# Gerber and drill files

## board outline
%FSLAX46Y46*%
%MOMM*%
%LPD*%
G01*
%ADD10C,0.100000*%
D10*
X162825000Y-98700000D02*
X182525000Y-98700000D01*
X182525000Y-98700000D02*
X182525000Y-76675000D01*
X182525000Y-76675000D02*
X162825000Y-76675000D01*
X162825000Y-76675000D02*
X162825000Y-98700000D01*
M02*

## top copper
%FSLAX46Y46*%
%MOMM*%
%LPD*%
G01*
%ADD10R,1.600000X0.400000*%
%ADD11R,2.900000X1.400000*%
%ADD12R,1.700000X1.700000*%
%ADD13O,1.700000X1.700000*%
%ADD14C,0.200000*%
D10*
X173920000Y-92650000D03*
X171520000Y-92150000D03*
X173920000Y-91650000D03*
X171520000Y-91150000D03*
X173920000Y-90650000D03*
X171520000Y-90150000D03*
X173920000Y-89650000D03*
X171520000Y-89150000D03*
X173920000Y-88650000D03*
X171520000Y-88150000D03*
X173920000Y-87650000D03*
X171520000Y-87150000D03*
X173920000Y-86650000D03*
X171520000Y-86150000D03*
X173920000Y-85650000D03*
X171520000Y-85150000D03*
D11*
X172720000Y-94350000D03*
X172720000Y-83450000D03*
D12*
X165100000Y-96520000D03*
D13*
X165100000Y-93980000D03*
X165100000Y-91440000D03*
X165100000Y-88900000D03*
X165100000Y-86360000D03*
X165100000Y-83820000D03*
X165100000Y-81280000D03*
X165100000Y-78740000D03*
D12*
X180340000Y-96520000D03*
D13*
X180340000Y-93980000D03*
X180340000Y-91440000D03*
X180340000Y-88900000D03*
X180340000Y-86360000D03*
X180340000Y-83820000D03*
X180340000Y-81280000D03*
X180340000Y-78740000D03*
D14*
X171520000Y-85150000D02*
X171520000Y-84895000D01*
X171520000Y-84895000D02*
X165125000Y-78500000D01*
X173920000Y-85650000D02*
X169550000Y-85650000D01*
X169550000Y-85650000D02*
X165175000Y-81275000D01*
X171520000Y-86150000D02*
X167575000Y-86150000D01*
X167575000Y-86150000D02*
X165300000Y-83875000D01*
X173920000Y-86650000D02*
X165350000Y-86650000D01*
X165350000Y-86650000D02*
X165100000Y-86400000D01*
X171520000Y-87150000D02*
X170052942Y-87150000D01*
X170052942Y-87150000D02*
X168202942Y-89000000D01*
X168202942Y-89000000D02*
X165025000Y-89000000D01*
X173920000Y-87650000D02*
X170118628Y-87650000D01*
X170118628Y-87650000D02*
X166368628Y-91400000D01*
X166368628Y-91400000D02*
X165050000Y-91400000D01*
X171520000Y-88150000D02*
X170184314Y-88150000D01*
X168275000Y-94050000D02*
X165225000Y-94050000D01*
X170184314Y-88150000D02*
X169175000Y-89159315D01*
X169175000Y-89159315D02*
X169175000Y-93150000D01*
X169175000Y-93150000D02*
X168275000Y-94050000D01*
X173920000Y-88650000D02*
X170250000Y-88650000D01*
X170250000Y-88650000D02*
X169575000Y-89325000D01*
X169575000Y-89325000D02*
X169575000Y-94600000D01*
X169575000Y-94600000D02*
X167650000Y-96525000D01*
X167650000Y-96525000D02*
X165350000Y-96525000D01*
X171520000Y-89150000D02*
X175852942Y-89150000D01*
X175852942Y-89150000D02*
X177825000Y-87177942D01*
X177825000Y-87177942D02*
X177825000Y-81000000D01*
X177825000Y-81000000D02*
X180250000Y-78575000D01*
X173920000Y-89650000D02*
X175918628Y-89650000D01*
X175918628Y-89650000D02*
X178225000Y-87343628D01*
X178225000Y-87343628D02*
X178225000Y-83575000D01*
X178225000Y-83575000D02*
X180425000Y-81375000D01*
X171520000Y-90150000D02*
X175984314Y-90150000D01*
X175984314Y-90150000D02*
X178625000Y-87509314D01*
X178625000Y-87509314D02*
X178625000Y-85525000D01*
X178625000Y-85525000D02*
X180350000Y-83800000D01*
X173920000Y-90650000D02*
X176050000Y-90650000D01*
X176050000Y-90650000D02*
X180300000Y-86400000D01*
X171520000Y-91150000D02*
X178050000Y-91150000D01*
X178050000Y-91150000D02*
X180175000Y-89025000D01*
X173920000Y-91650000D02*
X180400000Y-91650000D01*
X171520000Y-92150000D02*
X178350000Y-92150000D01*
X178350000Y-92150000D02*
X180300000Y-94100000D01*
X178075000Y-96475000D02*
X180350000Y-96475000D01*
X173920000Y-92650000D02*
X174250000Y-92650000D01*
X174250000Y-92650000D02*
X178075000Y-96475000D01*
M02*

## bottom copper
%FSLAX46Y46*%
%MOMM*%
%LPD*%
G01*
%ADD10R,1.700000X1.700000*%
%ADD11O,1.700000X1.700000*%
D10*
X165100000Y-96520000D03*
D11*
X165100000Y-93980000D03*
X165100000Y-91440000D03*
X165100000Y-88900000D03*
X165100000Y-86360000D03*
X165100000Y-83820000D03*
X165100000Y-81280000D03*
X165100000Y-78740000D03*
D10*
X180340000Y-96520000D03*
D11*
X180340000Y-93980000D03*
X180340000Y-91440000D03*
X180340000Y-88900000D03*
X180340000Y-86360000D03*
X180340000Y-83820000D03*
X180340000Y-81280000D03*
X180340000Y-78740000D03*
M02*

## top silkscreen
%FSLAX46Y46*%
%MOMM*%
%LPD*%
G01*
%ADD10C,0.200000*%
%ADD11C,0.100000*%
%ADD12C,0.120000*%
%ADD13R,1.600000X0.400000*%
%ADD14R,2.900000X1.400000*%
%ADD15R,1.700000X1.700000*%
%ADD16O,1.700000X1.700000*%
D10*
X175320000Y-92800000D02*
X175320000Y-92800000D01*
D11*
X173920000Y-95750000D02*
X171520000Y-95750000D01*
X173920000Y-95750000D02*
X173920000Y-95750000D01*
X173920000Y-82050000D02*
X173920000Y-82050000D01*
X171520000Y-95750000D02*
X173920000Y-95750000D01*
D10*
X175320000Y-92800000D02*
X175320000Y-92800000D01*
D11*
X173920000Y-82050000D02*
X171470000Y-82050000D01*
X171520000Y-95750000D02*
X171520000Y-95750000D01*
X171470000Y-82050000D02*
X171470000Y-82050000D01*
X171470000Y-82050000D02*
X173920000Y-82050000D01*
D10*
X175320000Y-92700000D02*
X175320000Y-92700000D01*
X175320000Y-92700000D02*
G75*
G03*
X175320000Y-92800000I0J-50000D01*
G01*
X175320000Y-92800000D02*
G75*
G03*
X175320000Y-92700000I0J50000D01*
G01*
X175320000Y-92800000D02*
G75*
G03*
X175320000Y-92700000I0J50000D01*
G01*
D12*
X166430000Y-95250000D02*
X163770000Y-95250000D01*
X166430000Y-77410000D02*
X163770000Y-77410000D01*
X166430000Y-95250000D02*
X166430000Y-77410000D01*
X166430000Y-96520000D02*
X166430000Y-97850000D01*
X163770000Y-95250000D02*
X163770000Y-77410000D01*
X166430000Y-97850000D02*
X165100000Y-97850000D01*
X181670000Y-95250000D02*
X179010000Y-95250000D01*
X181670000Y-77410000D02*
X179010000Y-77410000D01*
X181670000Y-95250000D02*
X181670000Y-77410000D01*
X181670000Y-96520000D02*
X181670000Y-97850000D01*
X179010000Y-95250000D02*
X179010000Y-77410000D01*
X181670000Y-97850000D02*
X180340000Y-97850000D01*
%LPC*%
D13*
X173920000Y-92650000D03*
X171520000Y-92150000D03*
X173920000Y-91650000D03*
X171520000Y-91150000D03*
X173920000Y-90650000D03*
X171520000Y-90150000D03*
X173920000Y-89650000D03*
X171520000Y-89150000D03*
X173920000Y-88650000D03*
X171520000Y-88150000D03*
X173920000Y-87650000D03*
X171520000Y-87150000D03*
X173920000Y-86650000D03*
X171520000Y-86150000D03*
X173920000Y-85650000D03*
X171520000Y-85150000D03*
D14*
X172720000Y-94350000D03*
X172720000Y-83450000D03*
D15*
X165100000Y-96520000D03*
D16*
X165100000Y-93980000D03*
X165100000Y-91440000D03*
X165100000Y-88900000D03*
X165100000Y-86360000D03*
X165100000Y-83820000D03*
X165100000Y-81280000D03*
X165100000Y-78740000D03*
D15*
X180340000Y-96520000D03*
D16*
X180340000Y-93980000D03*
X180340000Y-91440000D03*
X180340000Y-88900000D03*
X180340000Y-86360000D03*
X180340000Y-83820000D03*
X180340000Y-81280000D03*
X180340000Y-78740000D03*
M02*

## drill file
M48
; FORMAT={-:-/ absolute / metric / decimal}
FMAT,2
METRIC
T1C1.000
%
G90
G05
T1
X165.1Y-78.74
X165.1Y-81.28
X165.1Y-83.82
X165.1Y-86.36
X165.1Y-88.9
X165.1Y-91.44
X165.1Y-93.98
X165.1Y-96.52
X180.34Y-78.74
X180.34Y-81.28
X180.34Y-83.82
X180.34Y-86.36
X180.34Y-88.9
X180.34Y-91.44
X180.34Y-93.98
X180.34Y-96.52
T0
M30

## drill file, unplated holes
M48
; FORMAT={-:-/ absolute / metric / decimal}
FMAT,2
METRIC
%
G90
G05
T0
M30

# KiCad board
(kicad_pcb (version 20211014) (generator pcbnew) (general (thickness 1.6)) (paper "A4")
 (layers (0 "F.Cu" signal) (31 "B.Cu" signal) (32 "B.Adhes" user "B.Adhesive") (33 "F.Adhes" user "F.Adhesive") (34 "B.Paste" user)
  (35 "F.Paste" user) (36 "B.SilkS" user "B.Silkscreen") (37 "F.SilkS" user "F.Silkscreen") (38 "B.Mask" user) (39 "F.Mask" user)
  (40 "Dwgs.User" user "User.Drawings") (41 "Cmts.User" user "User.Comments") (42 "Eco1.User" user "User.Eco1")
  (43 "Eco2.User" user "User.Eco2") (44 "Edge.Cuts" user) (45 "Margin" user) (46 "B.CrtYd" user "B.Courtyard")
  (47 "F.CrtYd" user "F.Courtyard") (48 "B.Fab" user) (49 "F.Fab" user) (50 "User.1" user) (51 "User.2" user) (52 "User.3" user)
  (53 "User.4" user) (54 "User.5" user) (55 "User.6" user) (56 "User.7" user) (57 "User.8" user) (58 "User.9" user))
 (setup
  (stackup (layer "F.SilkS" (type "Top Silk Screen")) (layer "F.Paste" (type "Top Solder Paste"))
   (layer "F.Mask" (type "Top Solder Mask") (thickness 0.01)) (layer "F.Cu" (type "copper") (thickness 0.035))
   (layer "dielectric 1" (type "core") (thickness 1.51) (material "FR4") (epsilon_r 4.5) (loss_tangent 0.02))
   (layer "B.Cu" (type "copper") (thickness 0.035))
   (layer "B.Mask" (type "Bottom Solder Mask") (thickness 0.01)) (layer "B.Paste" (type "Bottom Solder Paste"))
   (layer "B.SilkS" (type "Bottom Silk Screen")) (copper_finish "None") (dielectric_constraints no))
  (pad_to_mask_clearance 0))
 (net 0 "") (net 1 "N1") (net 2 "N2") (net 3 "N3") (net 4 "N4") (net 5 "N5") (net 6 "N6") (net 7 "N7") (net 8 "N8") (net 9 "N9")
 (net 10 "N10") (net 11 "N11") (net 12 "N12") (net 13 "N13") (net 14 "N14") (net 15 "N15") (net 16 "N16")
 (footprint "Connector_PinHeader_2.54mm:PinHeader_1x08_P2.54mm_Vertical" (layer "F.Cu") (at 180.34 96.52 180)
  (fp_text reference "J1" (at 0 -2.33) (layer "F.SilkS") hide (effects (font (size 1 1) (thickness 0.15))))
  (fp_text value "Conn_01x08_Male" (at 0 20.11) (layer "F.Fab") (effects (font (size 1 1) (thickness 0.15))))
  (fp_line (start -1.33 -1.33) (end 0 -1.33) (layer "F.SilkS") (width 0.12))
  (fp_line (start -1.33 0) (end -1.33 -1.33) (layer "F.SilkS") (width 0.12))
  (fp_line (start -1.33 1.27) (end 1.33 1.27) (layer "F.SilkS") (width 0.12))
  (fp_line (start -1.33 1.27) (end -1.33 19.11) (layer "F.SilkS") (width 0.12))
  (fp_line (start 1.33 1.27) (end 1.33 19.11) (layer "F.SilkS") (width 0.12))
  (fp_line (start -1.33 19.11) (end 1.33 19.11) (layer "F.SilkS") (width 0.12))
  (pad "1" thru_hole rect (at 0 0 180) (size 1.7 1.7) (drill 1) (layers *.Cu *.Mask) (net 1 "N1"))
  (pad "2" thru_hole oval (at 0 2.54 180) (size 1.7 1.7) (drill 1) (layers *.Cu *.Mask) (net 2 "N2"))
  (pad "3" thru_hole oval (at 0 5.08 180) (size 1.7 1.7) (drill 1) (layers *.Cu *.Mask) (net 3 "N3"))
  (pad "4" thru_hole oval (at 0 7.62 180) (size 1.7 1.7) (drill 1) (layers *.Cu *.Mask) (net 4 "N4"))
  (pad "5" thru_hole oval (at 0 10.16 180) (size 1.7 1.7) (drill 1) (layers *.Cu *.Mask) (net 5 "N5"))
  (pad "6" thru_hole oval (at 0 12.7 180) (size 1.7 1.7) (drill 1) (layers *.Cu *.Mask) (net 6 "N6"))
  (pad "7" thru_hole oval (at 0 15.24 180) (size 1.7 1.7) (drill 1) (layers *.Cu *.Mask) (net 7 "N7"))
  (pad "8" thru_hole oval (at 0 17.78 180) (size 1.7 1.7) (drill 1) (layers *.Cu *.Mask) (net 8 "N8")))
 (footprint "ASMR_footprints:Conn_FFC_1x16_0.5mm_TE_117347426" (layer "F.Cu") (at 172.72 88.9 90)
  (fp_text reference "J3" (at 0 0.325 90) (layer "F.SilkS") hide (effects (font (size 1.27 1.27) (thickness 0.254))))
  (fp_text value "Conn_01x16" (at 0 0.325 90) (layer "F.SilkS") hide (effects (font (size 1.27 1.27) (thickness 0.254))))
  (fp_line (start -6.85 -1.2) (end -6.85 1.2) (layer "F.SilkS") (width 0.1))
  (fp_line (start -6.85 -1.2) (end -6.85 -1.2) (layer "F.SilkS") (width 0.1))
  (fp_line (start 6.85 -1.25) (end 6.85 1.2) (layer "F.SilkS") (width 0.1))
  (fp_line (start -3.9 2.6) (end -3.9 2.6) (layer "F.SilkS") (width 0.2))
  (fp_line (start -6.85 1.2) (end -6.85 -1.2) (layer "F.SilkS") (width 0.1))
  (fp_line (start 6.85 1.2) (end 6.85 1.2) (layer "F.SilkS") (width 0.1))
  (fp_line (start 6.85 1.2) (end 6.85 -1.25) (layer "F.SilkS") (width 0.1))
  (fp_line (start 6.85 -1.25) (end 6.85 -1.25) (layer "F.SilkS") (width 0.1))
  (fp_line (start -6.85 1.2) (end -6.85 1.2) (layer "F.SilkS") (width 0.1))
  (fp_line (start -3.9 2.6) (end -3.9 2.6) (layer "F.SilkS") (width 0.2))
  (fp_line (start -3.8 2.6) (end -3.8 2.6) (layer "F.SilkS") (width 0.2))
  (fp_arc (start -3.9 2.6) (mid -3.85 2.55) (end -3.8 2.6) (layer "F.SilkS") (width 0.2))
  (fp_arc (start -3.8 2.6) (mid -3.85 2.65) (end -3.9 2.6) (layer "F.SilkS") (width 0.2))
  (fp_arc (start -3.8 2.6) (mid -3.85 2.65) (end -3.9 2.6) (layer "F.SilkS") (width 0.2))
  (pad "1" smd rect (at -3.75 1.2 90) (size 0.4 1.6) (layers "F.Cu" "F.Paste" "F.Mask") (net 1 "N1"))
  (pad "2" smd rect (at -3.25 -1.2 90) (size 0.4 1.6) (layers "F.Cu" "F.Paste" "F.Mask") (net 2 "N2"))
  (pad "3" smd rect (at -2.75 1.2 90) (size 0.4 1.6) (layers "F.Cu" "F.Paste" "F.Mask") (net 3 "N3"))
  (pad "4" smd rect (at -2.25 -1.2 90) (size 0.4 1.6) (layers "F.Cu" "F.Paste" "F.Mask") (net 4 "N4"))
  (pad "5" smd rect (at -1.75 1.2 90) (size 0.4 1.6) (layers "F.Cu" "F.Paste" "F.Mask") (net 5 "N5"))
  (pad "6" smd rect (at -1.25 -1.2 90) (size 0.4 1.6) (layers "F.Cu" "F.Paste" "F.Mask") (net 6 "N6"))
  (pad "7" smd rect (at -0.75 1.2 90) (size 0.4 1.6) (layers "F.Cu" "F.Paste" "F.Mask") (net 7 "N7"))
  (pad "8" smd rect (at -0.25 -1.2 90) (size 0.4 1.6) (layers "F.Cu" "F.Paste" "F.Mask") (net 8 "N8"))
  (pad "9" smd rect (at 0.25 1.2 90) (size 0.4 1.6) (layers "F.Cu" "F.Paste" "F.Mask") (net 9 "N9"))
  (pad "10" smd rect (at 0.75 -1.2 90) (size 0.4 1.6) (layers "F.Cu" "F.Paste" "F.Mask") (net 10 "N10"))
  (pad "11" smd rect (at 1.25 1.2 90) (size 0.4 1.6) (layers "F.Cu" "F.Paste" "F.Mask") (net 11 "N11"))
  (pad "12" smd rect (at 1.75 -1.2 90) (size 0.4 1.6) (layers "F.Cu" "F.Paste" "F.Mask") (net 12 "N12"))
  (pad "13" smd rect (at 2.25 1.2 90) (size 0.4 1.6) (layers "F.Cu" "F.Paste" "F.Mask") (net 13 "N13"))
  (pad "14" smd rect (at 2.75 -1.2 90) (size 0.4 1.6) (layers "F.Cu" "F.Paste" "F.Mask") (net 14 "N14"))
  (pad "15" smd rect (at 3.25 1.2 90) (size 0.4 1.6) (layers "F.Cu" "F.Paste" "F.Mask") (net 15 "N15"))
  (pad "16" smd rect (at 3.75 -1.2 90) (size 0.4 1.6) (layers "F.Cu" "F.Paste" "F.Mask") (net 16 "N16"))
  (pad "MP1" smd rect (at -5.45 0 90) (size 1.4 2.9) (layers "F.Cu" "F.Paste" "F.Mask"))
  (pad "MP2" smd rect (at 5.45 0 90) (size 1.4 2.9) (layers "F.Cu" "F.Paste" "F.Mask")))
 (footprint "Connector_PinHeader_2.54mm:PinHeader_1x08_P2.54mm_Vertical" (layer "F.Cu") (at 165.1 96.52 180)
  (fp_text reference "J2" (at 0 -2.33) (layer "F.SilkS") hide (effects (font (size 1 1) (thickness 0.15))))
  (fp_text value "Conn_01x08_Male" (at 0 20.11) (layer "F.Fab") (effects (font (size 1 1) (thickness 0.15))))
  (fp_line (start -1.33 1.27) (end 1.33 1.27) (layer "F.SilkS") (width 0.12))
  (fp_line (start -1.33 19.11) (end 1.33 19.11) (layer "F.SilkS") (width 0.12))
  (fp_line (start -1.33 -1.33) (end 0 -1.33) (layer "F.SilkS") (width 0.12))
  (fp_line (start -1.33 0) (end -1.33 -1.33) (layer "F.SilkS") (width 0.12))
  (fp_line (start -1.33 1.27) (end -1.33 19.11) (layer "F.SilkS") (width 0.12))
  (fp_line (start 1.33 1.27) (end 1.33 19.11) (layer "F.SilkS") (width 0.12))
  (pad "1" thru_hole rect (at 0 0 180) (size 1.7 1.7) (drill 1) (layers *.Cu *.Mask) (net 9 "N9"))
  (pad "2" thru_hole oval (at 0 2.54 180) (size 1.7 1.7) (drill 1) (layers *.Cu *.Mask) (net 10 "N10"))
  (pad "3" thru_hole oval (at 0 5.08 180) (size 1.7 1.7) (drill 1) (layers *.Cu *.Mask) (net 11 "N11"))
  (pad "4" thru_hole oval (at 0 7.62 180) (size 1.7 1.7) (drill 1) (layers *.Cu *.Mask) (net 12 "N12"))
  (pad "5" thru_hole oval (at 0 10.16 180) (size 1.7 1.7) (drill 1) (layers *.Cu *.Mask) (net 13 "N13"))
  (pad "6" thru_hole oval (at 0 12.7 180) (size 1.7 1.7) (drill 1) (layers *.Cu *.Mask) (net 14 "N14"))
  (pad "7" thru_hole oval (at 0 15.24 180) (size 1.7 1.7) (drill 1) (layers *.Cu *.Mask) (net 15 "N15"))
  (pad "8" thru_hole oval (at 0 17.78 180) (size 1.7 1.7) (drill 1) (layers *.Cu *.Mask) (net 16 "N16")))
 (gr_rect (start 162.825 98.7) (end 182.525 76.675) (layer "Edge.Cuts") (width 0.1) (fill none))
 (segment (start 178.075 96.475) (end 180.35 96.475) (width 0.2) (layer "F.Cu") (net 1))
 (segment (start 173.92 92.65) (end 174.25 92.65) (width 0.2) (layer "F.Cu") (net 1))
 (segment (start 174.25 92.65) (end 178.075 96.475) (width 0.2) (layer "F.Cu") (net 1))
 (segment (start 171.52 92.15) (end 178.35 92.15) (width 0.2) (layer "F.Cu") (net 2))
 (segment (start 178.35 92.15) (end 180.3 94.1) (width 0.2) (layer "F.Cu") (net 2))
 (segment (start 173.92 91.65) (end 180.4 91.65) (width 0.2) (layer "F.Cu") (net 3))
 (segment (start 171.52 91.15) (end 178.05 91.15) (width 0.2) (layer "F.Cu") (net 4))
 (segment (start 178.05 91.15) (end 180.175 89.025) (width 0.2) (layer "F.Cu") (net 4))
 (segment (start 176.05 90.65) (end 180.3 86.4) (width 0.2) (layer "F.Cu") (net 5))
 (segment (start 173.92 90.65) (end 176.05 90.65) (width 0.2) (layer "F.Cu") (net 5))
 (segment (start 175.984314 90.15) (end 178.625 87.509314) (width 0.2) (layer "F.Cu") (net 6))
 (segment (start 171.52 90.15) (end 175.984314 90.15) (width 0.2) (layer "F.Cu") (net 6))
 (segment (start 178.625 85.525) (end 180.35 83.8) (width 0.2) (layer "F.Cu") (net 6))
 (segment (start 178.625 87.509314) (end 178.625 85.525) (width 0.2) (layer "F.Cu") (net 6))
 (segment (start 178.225 87.343628) (end 178.225 83.575) (width 0.2) (layer "F.Cu") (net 7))
 (segment (start 173.92 89.65) (end 175.918628 89.65) (width 0.2) (layer "F.Cu") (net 7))
 (segment (start 175.918628 89.65) (end 178.225 87.343628) (width 0.2) (layer "F.Cu") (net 7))
 (segment (start 178.225 83.575) (end 180.425 81.375) (width 0.2) (layer "F.Cu") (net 7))
 (segment (start 177.825 81) (end 180.25 78.575) (width 0.2) (layer "F.Cu") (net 8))
 (segment (start 177.825 87.177942) (end 177.825 81) (width 0.2) (layer "F.Cu") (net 8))
 (segment (start 171.52 89.15) (end 175.852942 89.15) (width 0.2) (layer "F.Cu") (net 8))
 (segment (start 175.852942 89.15) (end 177.825 87.177942) (width 0.2) (layer "F.Cu") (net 8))
 (segment (start 170.25 88.65) (end 169.575 89.325) (width 0.2) (layer "F.Cu") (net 9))
 (segment (start 169.575 89.325) (end 169.575 94.6) (width 0.2) (layer "F.Cu") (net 9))
 (segment (start 173.92 88.65) (end 170.25 88.65) (width 0.2) (layer "F.Cu") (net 9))
 (segment (start 167.65 96.525) (end 165.35 96.525) (width 0.2) (layer "F.Cu") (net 9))
 (segment (start 169.575 94.6) (end 167.65 96.525) (width 0.2) (layer "F.Cu") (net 9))
 (segment (start 169.175 93.15) (end 168.275 94.05) (width 0.2) (layer "F.Cu") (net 10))
 (segment (start 171.52 88.15) (end 170.184314 88.15) (width 0.2) (layer "F.Cu") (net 10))
 (segment (start 168.275 94.05) (end 165.225 94.05) (width 0.2) (layer "F.Cu") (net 10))
 (segment (start 170.184314 88.15) (end 169.175 89.159315) (width 0.2) (layer "F.Cu") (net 10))
 (segment (start 169.175 89.159315) (end 169.175 93.15) (width 0.2) (layer "F.Cu") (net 10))
 (segment (start 166.368628 91.4) (end 165.05 91.4) (width 0.2) (layer "F.Cu") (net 11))
 (segment (start 170.118628 87.65) (end 166.368628 91.4) (width 0.2) (layer "F.Cu") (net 11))
 (segment (start 173.92 87.65) (end 170.118628 87.65) (width 0.2) (layer "F.Cu") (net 11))
 (segment (start 171.52 87.15) (end 170.052942 87.15) (width 0.2) (layer "F.Cu") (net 12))
 (segment (start 170.052942 87.15) (end 168.202942 89) (width 0.2) (layer "F.Cu") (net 12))
 (segment (start 168.202942 89) (end 165.025 89) (width 0.2) (layer "F.Cu") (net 12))
 (segment (start 173.92 86.65) (end 165.35 86.65) (width 0.2) (layer "F.Cu") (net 13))
 (segment (start 165.35 86.65) (end 165.1 86.4) (width 0.2) (layer "F.Cu") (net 13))
 (segment (start 171.52 86.15) (end 167.575 86.15) (width 0.2) (layer "F.Cu") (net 14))
 (segment (start 167.575 86.15) (end 165.3 83.875) (width 0.2) (layer "F.Cu") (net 14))
 (segment (start 169.55 85.65) (end 165.175 81.275) (width 0.2) (layer "F.Cu") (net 15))
 (segment (start 173.92 85.65) (end 169.55 85.65) (width 0.2) (layer "F.Cu") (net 15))
 (segment (start 171.52 85.15) (end 171.52 84.895) (width 0.2) (layer "F.Cu") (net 16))
 (segment (start 171.52 84.895) (end 165.125 78.5) (width 0.2) (layer "F.Cu") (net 16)))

